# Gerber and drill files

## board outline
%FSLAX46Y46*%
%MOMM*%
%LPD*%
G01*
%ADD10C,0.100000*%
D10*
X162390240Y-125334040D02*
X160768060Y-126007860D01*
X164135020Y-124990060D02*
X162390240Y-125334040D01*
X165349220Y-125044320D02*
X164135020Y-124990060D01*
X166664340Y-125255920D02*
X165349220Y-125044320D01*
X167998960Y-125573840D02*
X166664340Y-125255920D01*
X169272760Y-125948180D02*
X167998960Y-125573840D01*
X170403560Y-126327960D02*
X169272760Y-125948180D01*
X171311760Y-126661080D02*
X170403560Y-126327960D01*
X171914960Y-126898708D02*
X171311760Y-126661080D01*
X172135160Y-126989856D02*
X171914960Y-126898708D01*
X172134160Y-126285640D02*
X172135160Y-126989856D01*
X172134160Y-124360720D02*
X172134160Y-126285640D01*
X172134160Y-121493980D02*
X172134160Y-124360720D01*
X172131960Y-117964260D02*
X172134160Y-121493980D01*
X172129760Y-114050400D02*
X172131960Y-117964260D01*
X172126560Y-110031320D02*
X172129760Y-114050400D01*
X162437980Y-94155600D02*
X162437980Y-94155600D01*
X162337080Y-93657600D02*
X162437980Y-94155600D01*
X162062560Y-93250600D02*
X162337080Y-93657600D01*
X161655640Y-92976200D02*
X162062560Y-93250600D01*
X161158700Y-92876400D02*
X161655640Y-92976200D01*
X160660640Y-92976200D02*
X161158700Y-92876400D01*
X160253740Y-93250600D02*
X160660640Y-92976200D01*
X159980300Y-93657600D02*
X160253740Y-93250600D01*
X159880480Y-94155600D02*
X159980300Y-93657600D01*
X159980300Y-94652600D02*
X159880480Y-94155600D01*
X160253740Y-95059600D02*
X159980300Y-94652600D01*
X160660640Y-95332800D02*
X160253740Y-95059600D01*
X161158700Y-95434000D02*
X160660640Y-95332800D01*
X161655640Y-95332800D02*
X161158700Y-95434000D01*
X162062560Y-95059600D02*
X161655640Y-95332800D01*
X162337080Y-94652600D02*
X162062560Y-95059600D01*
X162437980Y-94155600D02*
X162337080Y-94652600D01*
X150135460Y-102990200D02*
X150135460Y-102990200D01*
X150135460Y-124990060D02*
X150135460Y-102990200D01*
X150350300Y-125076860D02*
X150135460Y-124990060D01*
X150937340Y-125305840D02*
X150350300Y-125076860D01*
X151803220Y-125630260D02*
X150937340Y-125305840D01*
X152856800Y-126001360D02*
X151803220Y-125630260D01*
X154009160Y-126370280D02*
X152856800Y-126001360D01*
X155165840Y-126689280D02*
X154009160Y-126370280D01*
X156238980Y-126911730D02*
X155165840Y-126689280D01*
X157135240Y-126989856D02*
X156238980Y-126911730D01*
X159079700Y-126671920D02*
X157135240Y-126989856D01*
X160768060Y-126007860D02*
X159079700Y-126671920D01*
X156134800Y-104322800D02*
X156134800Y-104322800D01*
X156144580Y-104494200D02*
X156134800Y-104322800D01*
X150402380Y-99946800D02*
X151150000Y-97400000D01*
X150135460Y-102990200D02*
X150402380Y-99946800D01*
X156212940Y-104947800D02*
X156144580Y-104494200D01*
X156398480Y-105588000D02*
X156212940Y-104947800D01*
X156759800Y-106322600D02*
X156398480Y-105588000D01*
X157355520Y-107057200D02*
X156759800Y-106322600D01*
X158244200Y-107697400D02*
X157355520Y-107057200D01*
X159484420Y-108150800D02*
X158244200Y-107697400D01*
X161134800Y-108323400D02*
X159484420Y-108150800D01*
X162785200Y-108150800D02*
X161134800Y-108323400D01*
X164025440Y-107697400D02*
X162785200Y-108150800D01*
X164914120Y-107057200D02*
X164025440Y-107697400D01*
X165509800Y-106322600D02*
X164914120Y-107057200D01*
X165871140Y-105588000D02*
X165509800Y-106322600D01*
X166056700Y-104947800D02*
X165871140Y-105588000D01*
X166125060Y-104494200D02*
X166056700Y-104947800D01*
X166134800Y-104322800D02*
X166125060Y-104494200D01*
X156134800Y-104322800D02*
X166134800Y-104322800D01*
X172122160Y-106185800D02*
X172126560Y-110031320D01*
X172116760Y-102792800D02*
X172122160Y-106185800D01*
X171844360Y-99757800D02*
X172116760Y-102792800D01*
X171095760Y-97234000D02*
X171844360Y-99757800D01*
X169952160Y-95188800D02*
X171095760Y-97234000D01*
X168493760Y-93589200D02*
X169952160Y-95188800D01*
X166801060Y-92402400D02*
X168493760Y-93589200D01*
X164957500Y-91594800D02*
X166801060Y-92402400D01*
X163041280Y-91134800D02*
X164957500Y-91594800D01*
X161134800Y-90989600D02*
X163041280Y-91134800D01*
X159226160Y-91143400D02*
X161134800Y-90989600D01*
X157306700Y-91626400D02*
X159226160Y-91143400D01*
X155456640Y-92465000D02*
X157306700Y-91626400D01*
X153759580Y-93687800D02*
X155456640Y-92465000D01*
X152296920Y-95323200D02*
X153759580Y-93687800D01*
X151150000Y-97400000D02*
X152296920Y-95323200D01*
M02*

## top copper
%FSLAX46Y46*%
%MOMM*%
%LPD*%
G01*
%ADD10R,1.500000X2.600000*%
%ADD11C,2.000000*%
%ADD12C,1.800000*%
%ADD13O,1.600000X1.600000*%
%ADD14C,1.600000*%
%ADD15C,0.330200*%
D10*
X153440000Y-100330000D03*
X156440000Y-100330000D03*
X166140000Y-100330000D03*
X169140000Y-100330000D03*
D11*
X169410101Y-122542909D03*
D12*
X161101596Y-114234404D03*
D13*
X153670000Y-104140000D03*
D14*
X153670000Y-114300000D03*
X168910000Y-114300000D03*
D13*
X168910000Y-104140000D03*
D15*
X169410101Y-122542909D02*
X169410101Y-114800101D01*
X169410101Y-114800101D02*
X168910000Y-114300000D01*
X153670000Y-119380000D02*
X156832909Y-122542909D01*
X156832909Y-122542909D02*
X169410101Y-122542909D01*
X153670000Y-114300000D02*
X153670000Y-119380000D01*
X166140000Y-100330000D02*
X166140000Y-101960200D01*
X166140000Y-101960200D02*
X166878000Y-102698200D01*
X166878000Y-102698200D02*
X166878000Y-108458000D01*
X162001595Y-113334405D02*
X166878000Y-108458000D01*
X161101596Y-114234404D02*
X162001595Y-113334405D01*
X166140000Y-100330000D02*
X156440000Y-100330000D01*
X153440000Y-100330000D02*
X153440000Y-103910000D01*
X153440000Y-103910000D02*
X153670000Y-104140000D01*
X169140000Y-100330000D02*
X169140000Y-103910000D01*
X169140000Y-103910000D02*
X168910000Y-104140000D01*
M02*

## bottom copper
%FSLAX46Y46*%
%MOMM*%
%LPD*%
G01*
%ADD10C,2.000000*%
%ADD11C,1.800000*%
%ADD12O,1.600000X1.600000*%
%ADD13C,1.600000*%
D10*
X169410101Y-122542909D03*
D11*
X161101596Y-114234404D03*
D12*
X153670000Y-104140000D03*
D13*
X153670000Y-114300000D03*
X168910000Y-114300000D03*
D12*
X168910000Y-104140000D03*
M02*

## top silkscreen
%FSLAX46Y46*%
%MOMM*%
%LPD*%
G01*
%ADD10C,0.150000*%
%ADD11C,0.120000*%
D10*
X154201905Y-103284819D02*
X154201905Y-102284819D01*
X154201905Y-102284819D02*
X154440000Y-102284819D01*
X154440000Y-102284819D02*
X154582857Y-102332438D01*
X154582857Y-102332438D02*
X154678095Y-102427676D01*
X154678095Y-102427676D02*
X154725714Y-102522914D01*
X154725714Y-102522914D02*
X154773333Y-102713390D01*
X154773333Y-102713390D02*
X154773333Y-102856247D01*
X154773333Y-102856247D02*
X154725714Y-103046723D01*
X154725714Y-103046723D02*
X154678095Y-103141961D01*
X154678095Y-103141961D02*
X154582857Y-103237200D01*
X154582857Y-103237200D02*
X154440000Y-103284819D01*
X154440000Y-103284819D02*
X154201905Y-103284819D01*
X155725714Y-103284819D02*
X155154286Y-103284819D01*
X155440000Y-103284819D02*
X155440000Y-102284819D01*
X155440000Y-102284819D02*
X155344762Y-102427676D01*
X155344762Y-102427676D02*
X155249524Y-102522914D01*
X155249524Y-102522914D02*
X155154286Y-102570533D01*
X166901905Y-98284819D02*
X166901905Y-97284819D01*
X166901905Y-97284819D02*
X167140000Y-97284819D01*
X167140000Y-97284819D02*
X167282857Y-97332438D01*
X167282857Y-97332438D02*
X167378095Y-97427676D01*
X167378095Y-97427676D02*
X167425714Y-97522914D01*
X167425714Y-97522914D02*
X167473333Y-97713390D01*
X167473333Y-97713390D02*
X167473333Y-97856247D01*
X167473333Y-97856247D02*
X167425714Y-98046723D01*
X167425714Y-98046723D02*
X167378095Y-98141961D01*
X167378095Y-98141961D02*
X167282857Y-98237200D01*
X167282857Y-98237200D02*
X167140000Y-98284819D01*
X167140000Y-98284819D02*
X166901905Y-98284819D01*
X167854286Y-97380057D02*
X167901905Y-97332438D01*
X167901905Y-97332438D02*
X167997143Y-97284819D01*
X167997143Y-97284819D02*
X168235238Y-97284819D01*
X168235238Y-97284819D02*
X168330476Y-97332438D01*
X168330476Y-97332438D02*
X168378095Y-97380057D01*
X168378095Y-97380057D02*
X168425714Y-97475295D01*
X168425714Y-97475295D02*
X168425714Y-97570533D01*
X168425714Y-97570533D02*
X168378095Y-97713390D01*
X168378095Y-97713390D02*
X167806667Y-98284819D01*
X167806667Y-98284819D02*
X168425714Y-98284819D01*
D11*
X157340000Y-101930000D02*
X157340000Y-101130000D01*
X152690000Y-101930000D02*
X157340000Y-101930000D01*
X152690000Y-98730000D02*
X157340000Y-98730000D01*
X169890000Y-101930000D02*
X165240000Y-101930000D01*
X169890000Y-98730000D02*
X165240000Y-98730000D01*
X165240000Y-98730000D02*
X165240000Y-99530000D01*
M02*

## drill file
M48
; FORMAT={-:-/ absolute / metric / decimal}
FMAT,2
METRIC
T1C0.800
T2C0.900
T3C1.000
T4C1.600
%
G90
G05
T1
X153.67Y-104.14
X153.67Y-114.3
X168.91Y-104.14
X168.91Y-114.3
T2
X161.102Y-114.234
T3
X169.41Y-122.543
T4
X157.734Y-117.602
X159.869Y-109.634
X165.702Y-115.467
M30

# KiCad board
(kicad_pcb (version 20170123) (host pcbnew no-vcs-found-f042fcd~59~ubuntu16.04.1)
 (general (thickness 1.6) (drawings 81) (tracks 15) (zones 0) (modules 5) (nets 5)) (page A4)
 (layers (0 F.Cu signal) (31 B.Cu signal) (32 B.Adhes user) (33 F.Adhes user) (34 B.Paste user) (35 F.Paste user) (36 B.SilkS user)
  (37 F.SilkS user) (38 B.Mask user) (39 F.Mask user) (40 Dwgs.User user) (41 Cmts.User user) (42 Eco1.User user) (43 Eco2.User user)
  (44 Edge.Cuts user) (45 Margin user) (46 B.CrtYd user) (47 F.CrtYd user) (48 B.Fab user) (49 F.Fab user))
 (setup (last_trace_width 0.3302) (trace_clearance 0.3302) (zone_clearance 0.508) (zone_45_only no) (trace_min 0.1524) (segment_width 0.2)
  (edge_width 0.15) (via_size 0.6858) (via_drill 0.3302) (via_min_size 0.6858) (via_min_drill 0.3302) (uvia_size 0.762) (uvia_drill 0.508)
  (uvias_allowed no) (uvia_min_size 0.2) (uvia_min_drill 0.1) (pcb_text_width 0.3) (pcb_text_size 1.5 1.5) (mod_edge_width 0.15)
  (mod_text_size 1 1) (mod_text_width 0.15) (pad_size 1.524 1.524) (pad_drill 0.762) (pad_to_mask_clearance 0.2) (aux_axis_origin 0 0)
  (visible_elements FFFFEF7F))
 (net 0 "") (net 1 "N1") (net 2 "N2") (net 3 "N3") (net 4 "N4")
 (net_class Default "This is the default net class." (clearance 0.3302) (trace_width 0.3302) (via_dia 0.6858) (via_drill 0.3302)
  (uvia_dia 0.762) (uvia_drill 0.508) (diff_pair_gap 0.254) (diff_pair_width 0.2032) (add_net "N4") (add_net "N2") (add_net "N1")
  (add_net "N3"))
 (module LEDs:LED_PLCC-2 (layer F.Cu) (at 154.94 100.33 180)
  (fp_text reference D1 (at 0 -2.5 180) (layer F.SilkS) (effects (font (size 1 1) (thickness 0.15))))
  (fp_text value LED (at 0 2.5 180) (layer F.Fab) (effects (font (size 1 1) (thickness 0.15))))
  (fp_line (start -2.4 -1.6) (end -2.4 -0.8) (layer F.SilkS) (width 0.12))
  (fp_line (start 2.25 -1.6) (end -2.4 -1.6) (layer F.SilkS) (width 0.12))
  (fp_line (start 2.25 1.6) (end -2.4 1.6) (layer F.SilkS) (width 0.12))
  (pad 2 smd rect (at 1.5 0 180) (size 1.5 2.6) (layers F.Cu F.Paste F.Mask) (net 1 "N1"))
  (pad 1 smd rect (at -1.5 0 180) (size 1.5 2.6) (layers F.Cu F.Paste F.Mask) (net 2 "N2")))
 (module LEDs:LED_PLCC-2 (layer F.Cu) (at 167.64 100.33)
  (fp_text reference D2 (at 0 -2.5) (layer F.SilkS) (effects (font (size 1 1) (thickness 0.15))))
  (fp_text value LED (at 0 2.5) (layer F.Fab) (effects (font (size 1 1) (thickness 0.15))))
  (fp_line (start 2.25 1.6) (end -2.4 1.6) (layer F.SilkS) (width 0.12))
  (fp_line (start 2.25 -1.6) (end -2.4 -1.6) (layer F.SilkS) (width 0.12))
  (fp_line (start -2.4 -1.6) (end -2.4 -0.8) (layer F.SilkS) (width 0.12))
  (pad 1 smd rect (at -1.5 0) (size 1.5 2.6) (layers F.Cu F.Paste F.Mask) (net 2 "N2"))
  (pad 2 smd rect (at 1.5 0) (size 1.5 2.6) (layers F.Cu F.Paste F.Mask) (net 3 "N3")))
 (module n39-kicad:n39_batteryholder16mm (layer B.Cu) (at 161.101596 114.234404 315)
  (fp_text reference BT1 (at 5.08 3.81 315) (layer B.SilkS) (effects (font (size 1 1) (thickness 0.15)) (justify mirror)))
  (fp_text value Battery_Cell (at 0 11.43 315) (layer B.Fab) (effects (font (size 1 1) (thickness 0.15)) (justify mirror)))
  (pad "" np_thru_hole circle (at 0 4.7625 315) (size 1.6 1.6) (drill 1.6) (layers *.Cu *.Mask))
  (pad 1 thru_hole circle (at 11.75 0 315) (size 2 2) (drill 1) (layers *.Cu *.Mask) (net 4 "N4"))
  (pad 2 thru_hole circle (at 0 0 315) (size 1.8 1.8) (drill 0.9) (layers *.Cu *.Mask) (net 2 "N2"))
  (pad "" np_thru_hole circle (at -4.124446 -2.38125 195) (size 1.6 1.6) (drill 1.6) (layers *.Cu *.Mask))
  (pad "" np_thru_hole circle (at 4.124446 -2.38125 75) (size 1.6 1.6) (drill 1.6) (layers *.Cu *.Mask)))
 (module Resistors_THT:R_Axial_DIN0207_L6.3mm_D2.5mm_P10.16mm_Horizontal (layer B.Cu) (at 153.67 114.3 90)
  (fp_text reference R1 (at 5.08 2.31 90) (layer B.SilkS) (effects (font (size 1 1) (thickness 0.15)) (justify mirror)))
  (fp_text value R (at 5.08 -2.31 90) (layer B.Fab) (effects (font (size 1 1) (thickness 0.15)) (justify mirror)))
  (pad 2 thru_hole oval (at 10.16 0 90) (size 1.6 1.6) (drill 0.8) (layers *.Cu *.Mask) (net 1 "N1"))
  (pad 1 thru_hole circle (at 0 0 90) (size 1.6 1.6) (drill 0.8) (layers *.Cu *.Mask) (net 4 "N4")))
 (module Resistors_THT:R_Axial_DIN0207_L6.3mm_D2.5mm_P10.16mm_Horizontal (layer B.Cu) (at 168.91 114.3 90)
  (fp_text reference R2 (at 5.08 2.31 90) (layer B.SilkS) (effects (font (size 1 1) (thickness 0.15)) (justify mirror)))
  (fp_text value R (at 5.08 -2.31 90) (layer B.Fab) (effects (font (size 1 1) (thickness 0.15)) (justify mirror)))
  (pad 1 thru_hole circle (at 0 0 90) (size 1.6 1.6) (drill 0.8) (layers *.Cu *.Mask) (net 4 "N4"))
  (pad 2 thru_hole oval (at 10.16 0 90) (size 1.6 1.6) (drill 0.8) (layers *.Cu *.Mask) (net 3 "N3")))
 (gr_line (start 162.39024 125.33404) (end 160.76806 126.00786) (layer Edge.Cuts) (width 0.1))
 (gr_line (start 164.13502 124.99006) (end 162.39024 125.33404) (layer Edge.Cuts) (width 0.1))
 (gr_line (start 165.34922 125.04432) (end 164.13502 124.99006) (layer Edge.Cuts) (width 0.1))
 (gr_line (start 166.66434 125.25592) (end 165.34922 125.04432) (layer Edge.Cuts) (width 0.1))
 (gr_line (start 167.99896 125.57384) (end 166.66434 125.25592) (layer Edge.Cuts) (width 0.1))
 (gr_line (start 169.27276 125.94818) (end 167.99896 125.57384) (layer Edge.Cuts) (width 0.1))
 (gr_line (start 170.40356 126.32796) (end 169.27276 125.94818) (layer Edge.Cuts) (width 0.1))
 (gr_line (start 171.31176 126.66108) (end 170.40356 126.32796) (layer Edge.Cuts) (width 0.1))
 (gr_line (start 171.91496 126.898708) (end 171.31176 126.66108) (layer Edge.Cuts) (width 0.1))
 (gr_line (start 172.13516 126.989856) (end 171.91496 126.898708) (layer Edge.Cuts) (width 0.1))
 (gr_line (start 172.13416 126.28564) (end 172.13516 126.989856) (layer Edge.Cuts) (width 0.1))
 (gr_line (start 172.13416 124.36072) (end 172.13416 126.28564) (layer Edge.Cuts) (width 0.1))
 (gr_line (start 172.13416 121.49398) (end 172.13416 124.36072) (layer Edge.Cuts) (width 0.1))
 (gr_line (start 172.13196 117.96426) (end 172.13416 121.49398) (layer Edge.Cuts) (width 0.1))
 (gr_line (start 172.12976 114.0504) (end 172.13196 117.96426) (layer Edge.Cuts) (width 0.1))
 (gr_line (start 172.12656 110.03132) (end 172.12976 114.0504) (layer Edge.Cuts) (width 0.1))
 (gr_line (start 162.43798 94.1556) (end 162.43798 94.1556) (layer Edge.Cuts) (width 0.1))
 (gr_line (start 162.33708 93.6576) (end 162.43798 94.1556) (layer Edge.Cuts) (width 0.1))
 (gr_line (start 162.06256 93.2506) (end 162.33708 93.6576) (layer Edge.Cuts) (width 0.1))
 (gr_line (start 161.65564 92.9762) (end 162.06256 93.2506) (layer Edge.Cuts) (width 0.1))
 (gr_line (start 161.1587 92.8764) (end 161.65564 92.9762) (layer Edge.Cuts) (width 0.1))
 (gr_line (start 160.66064 92.9762) (end 161.1587 92.8764) (layer Edge.Cuts) (width 0.1))
 (gr_line (start 160.25374 93.2506) (end 160.66064 92.9762) (layer Edge.Cuts) (width 0.1))
 (gr_line (start 159.9803 93.6576) (end 160.25374 93.2506) (layer Edge.Cuts) (width 0.1))
 (gr_line (start 159.88048 94.1556) (end 159.9803 93.6576) (layer Edge.Cuts) (width 0.1))
 (gr_line (start 159.9803 94.6526) (end 159.88048 94.1556) (layer Edge.Cuts) (width 0.1))
 (gr_line (start 160.25374 95.0596) (end 159.9803 94.6526) (layer Edge.Cuts) (width 0.1))
 (gr_line (start 160.66064 95.3328) (end 160.25374 95.0596) (layer Edge.Cuts) (width 0.1))
 (gr_line (start 161.1587 95.434) (end 160.66064 95.3328) (layer Edge.Cuts) (width 0.1))
 (gr_line (start 161.65564 95.3328) (end 161.1587 95.434) (layer Edge.Cuts) (width 0.1))
 (gr_line (start 162.06256 95.0596) (end 161.65564 95.3328) (layer Edge.Cuts) (width 0.1))
 (gr_line (start 162.33708 94.6526) (end 162.06256 95.0596) (layer Edge.Cuts) (width 0.1))
 (gr_line (start 162.43798 94.1556) (end 162.33708 94.6526) (layer Edge.Cuts) (width 0.1))
 (gr_line (start 150.13546 102.9902) (end 150.13546 102.9902) (layer Edge.Cuts) (width 0.1))
 (gr_line (start 150.13546 124.99006) (end 150.13546 102.9902) (layer Edge.Cuts) (width 0.1))
 (gr_line (start 150.3503 125.07686) (end 150.13546 124.99006) (layer Edge.Cuts) (width 0.1))
 (gr_line (start 150.93734 125.30584) (end 150.3503 125.07686) (layer Edge.Cuts) (width 0.1))
 (gr_line (start 151.80322 125.63026) (end 150.93734 125.30584) (layer Edge.Cuts) (width 0.1))
 (gr_line (start 152.8568 126.00136) (end 151.80322 125.63026) (layer Edge.Cuts) (width 0.1))
 (gr_line (start 154.00916 126.37028) (end 152.8568 126.00136) (layer Edge.Cuts) (width 0.1))
 (gr_line (start 155.16584 126.68928) (end 154.00916 126.37028) (layer Edge.Cuts) (width 0.1))
 (gr_line (start 156.23898 126.91173) (end 155.16584 126.68928) (layer Edge.Cuts) (width 0.1))
 (gr_line (start 157.13524 126.989856) (end 156.23898 126.91173) (layer Edge.Cuts) (width 0.1))
 (gr_line (start 159.0797 126.67192) (end 157.13524 126.989856) (layer Edge.Cuts) (width 0.1))
 (gr_line (start 160.76806 126.00786) (end 159.0797 126.67192) (layer Edge.Cuts) (width 0.1))
 (gr_line (start 156.1348 104.3228) (end 156.1348 104.3228) (layer Edge.Cuts) (width 0.1))
 (gr_line (start 156.14458 104.4942) (end 156.1348 104.3228) (layer Edge.Cuts) (width 0.1))
 (gr_line (start 150.40238 99.9468) (end 151.15 97.4) (layer Edge.Cuts) (width 0.1))
 (gr_line (start 150.13546 102.9902) (end 150.40238 99.9468) (layer Edge.Cuts) (width 0.1))
 (gr_line (start 156.21294 104.9478) (end 156.14458 104.4942) (layer Edge.Cuts) (width 0.1))
 (gr_line (start 156.39848 105.588) (end 156.21294 104.9478) (layer Edge.Cuts) (width 0.1))
 (gr_line (start 156.7598 106.3226) (end 156.39848 105.588) (layer Edge.Cuts) (width 0.1))
 (gr_line (start 157.35552 107.0572) (end 156.7598 106.3226) (layer Edge.Cuts) (width 0.1))
 (gr_line (start 158.2442 107.6974) (end 157.35552 107.0572) (layer Edge.Cuts) (width 0.1))
 (gr_line (start 159.48442 108.1508) (end 158.2442 107.6974) (layer Edge.Cuts) (width 0.1))
 (gr_line (start 161.1348 108.3234) (end 159.48442 108.1508) (layer Edge.Cuts) (width 0.1))
 (gr_line (start 162.7852 108.1508) (end 161.1348 108.3234) (layer Edge.Cuts) (width 0.1))
 (gr_line (start 164.02544 107.6974) (end 162.7852 108.1508) (layer Edge.Cuts) (width 0.1))
 (gr_line (start 164.91412 107.0572) (end 164.02544 107.6974) (layer Edge.Cuts) (width 0.1))
 (gr_line (start 165.5098 106.3226) (end 164.91412 107.0572) (layer Edge.Cuts) (width 0.1))
 (gr_line (start 165.87114 105.588) (end 165.5098 106.3226) (layer Edge.Cuts) (width 0.1))
 (gr_line (start 166.0567 104.9478) (end 165.87114 105.588) (layer Edge.Cuts) (width 0.1))
 (gr_line (start 166.12506 104.4942) (end 166.0567 104.9478) (layer Edge.Cuts) (width 0.1))
 (gr_line (start 166.1348 104.3228) (end 166.12506 104.4942) (layer Edge.Cuts) (width 0.1))
 (gr_line (start 156.1348 104.3228) (end 166.1348 104.3228) (layer Edge.Cuts) (width 0.1))
 (gr_line (start 172.12216 106.1858) (end 172.12656 110.03132) (layer Edge.Cuts) (width 0.1))
 (gr_line (start 172.11676 102.7928) (end 172.12216 106.1858) (layer Edge.Cuts) (width 0.1))
 (gr_line (start 171.84436 99.7578) (end 172.11676 102.7928) (layer Edge.Cuts) (width 0.1))
 (gr_line (start 171.09576 97.234) (end 171.84436 99.7578) (layer Edge.Cuts) (width 0.1))
 (gr_line (start 169.95216 95.1888) (end 171.09576 97.234) (layer Edge.Cuts) (width 0.1))
 (gr_line (start 168.49376 93.5892) (end 169.95216 95.1888) (layer Edge.Cuts) (width 0.1))
 (gr_line (start 166.80106 92.4024) (end 168.49376 93.5892) (layer Edge.Cuts) (width 0.1))
 (gr_line (start 164.9575 91.5948) (end 166.80106 92.4024) (layer Edge.Cuts) (width 0.1))
 (gr_line (start 163.04128 91.1348) (end 164.9575 91.5948) (layer Edge.Cuts) (width 0.1))
 (gr_line (start 161.1348 90.9896) (end 163.04128 91.1348) (layer Edge.Cuts) (width 0.1))
 (gr_line (start 159.22616 91.1434) (end 161.1348 90.9896) (layer Edge.Cuts) (width 0.1))
 (gr_line (start 157.3067 91.6264) (end 159.22616 91.1434) (layer Edge.Cuts) (width 0.1))
 (gr_line (start 155.45664 92.465) (end 157.3067 91.6264) (layer Edge.Cuts) (width 0.1))
 (gr_line (start 153.75958 93.6878) (end 155.45664 92.465) (layer Edge.Cuts) (width 0.1))
 (gr_line (start 152.29692 95.3232) (end 153.75958 93.6878) (layer Edge.Cuts) (width 0.1))
 (gr_line (start 151.15 97.4) (end 152.29692 95.3232) (layer Edge.Cuts) (width 0.1))
 (segment (start 169.410101 122.542909) (end 169.410101 114.800101) (width 0.3302) (layer F.Cu) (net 4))
 (segment (start 169.410101 114.800101) (end 168.91 114.3) (width 0.3302) (layer F.Cu) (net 4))
 (segment (start 153.67 119.38) (end 156.832909 122.542909) (width 0.3302) (layer F.Cu) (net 4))
 (segment (start 156.832909 122.542909) (end 169.410101 122.542909) (width 0.3302) (layer F.Cu) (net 4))
 (segment (start 153.67 114.3) (end 153.67 119.38) (width 0.3302) (layer F.Cu) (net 4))
 (segment (start 166.14 100.33) (end 166.14 101.9602) (width 0.3302) (layer F.Cu) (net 2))
 (segment (start 166.14 101.9602) (end 166.878 102.6982) (width 0.3302) (layer F.Cu) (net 2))
 (segment (start 166.878 102.6982) (end 166.878 108.458) (width 0.3302) (layer F.Cu) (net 2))
 (segment (start 162.001595 113.334405) (end 166.878 108.458) (width 0.3302) (layer F.Cu) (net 2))
 (segment (start 161.101596 114.234404) (end 162.001595 113.334405) (width 0.3302) (layer F.Cu) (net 2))
 (segment (start 166.14 100.33) (end 156.44 100.33) (width 0.3302) (layer F.Cu) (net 2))
 (segment (start 153.44 100.33) (end 153.44 103.91) (width 0.3302) (layer F.Cu) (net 1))
 (segment (start 153.44 103.91) (end 153.67 104.14) (width 0.3302) (layer F.Cu) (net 1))
 (segment (start 169.14 100.33) (end 169.14 103.91) (width 0.3302) (layer F.Cu) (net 3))
 (segment (start 169.14 103.91) (end 168.91 104.14) (width 0.3302) (layer F.Cu) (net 3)))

